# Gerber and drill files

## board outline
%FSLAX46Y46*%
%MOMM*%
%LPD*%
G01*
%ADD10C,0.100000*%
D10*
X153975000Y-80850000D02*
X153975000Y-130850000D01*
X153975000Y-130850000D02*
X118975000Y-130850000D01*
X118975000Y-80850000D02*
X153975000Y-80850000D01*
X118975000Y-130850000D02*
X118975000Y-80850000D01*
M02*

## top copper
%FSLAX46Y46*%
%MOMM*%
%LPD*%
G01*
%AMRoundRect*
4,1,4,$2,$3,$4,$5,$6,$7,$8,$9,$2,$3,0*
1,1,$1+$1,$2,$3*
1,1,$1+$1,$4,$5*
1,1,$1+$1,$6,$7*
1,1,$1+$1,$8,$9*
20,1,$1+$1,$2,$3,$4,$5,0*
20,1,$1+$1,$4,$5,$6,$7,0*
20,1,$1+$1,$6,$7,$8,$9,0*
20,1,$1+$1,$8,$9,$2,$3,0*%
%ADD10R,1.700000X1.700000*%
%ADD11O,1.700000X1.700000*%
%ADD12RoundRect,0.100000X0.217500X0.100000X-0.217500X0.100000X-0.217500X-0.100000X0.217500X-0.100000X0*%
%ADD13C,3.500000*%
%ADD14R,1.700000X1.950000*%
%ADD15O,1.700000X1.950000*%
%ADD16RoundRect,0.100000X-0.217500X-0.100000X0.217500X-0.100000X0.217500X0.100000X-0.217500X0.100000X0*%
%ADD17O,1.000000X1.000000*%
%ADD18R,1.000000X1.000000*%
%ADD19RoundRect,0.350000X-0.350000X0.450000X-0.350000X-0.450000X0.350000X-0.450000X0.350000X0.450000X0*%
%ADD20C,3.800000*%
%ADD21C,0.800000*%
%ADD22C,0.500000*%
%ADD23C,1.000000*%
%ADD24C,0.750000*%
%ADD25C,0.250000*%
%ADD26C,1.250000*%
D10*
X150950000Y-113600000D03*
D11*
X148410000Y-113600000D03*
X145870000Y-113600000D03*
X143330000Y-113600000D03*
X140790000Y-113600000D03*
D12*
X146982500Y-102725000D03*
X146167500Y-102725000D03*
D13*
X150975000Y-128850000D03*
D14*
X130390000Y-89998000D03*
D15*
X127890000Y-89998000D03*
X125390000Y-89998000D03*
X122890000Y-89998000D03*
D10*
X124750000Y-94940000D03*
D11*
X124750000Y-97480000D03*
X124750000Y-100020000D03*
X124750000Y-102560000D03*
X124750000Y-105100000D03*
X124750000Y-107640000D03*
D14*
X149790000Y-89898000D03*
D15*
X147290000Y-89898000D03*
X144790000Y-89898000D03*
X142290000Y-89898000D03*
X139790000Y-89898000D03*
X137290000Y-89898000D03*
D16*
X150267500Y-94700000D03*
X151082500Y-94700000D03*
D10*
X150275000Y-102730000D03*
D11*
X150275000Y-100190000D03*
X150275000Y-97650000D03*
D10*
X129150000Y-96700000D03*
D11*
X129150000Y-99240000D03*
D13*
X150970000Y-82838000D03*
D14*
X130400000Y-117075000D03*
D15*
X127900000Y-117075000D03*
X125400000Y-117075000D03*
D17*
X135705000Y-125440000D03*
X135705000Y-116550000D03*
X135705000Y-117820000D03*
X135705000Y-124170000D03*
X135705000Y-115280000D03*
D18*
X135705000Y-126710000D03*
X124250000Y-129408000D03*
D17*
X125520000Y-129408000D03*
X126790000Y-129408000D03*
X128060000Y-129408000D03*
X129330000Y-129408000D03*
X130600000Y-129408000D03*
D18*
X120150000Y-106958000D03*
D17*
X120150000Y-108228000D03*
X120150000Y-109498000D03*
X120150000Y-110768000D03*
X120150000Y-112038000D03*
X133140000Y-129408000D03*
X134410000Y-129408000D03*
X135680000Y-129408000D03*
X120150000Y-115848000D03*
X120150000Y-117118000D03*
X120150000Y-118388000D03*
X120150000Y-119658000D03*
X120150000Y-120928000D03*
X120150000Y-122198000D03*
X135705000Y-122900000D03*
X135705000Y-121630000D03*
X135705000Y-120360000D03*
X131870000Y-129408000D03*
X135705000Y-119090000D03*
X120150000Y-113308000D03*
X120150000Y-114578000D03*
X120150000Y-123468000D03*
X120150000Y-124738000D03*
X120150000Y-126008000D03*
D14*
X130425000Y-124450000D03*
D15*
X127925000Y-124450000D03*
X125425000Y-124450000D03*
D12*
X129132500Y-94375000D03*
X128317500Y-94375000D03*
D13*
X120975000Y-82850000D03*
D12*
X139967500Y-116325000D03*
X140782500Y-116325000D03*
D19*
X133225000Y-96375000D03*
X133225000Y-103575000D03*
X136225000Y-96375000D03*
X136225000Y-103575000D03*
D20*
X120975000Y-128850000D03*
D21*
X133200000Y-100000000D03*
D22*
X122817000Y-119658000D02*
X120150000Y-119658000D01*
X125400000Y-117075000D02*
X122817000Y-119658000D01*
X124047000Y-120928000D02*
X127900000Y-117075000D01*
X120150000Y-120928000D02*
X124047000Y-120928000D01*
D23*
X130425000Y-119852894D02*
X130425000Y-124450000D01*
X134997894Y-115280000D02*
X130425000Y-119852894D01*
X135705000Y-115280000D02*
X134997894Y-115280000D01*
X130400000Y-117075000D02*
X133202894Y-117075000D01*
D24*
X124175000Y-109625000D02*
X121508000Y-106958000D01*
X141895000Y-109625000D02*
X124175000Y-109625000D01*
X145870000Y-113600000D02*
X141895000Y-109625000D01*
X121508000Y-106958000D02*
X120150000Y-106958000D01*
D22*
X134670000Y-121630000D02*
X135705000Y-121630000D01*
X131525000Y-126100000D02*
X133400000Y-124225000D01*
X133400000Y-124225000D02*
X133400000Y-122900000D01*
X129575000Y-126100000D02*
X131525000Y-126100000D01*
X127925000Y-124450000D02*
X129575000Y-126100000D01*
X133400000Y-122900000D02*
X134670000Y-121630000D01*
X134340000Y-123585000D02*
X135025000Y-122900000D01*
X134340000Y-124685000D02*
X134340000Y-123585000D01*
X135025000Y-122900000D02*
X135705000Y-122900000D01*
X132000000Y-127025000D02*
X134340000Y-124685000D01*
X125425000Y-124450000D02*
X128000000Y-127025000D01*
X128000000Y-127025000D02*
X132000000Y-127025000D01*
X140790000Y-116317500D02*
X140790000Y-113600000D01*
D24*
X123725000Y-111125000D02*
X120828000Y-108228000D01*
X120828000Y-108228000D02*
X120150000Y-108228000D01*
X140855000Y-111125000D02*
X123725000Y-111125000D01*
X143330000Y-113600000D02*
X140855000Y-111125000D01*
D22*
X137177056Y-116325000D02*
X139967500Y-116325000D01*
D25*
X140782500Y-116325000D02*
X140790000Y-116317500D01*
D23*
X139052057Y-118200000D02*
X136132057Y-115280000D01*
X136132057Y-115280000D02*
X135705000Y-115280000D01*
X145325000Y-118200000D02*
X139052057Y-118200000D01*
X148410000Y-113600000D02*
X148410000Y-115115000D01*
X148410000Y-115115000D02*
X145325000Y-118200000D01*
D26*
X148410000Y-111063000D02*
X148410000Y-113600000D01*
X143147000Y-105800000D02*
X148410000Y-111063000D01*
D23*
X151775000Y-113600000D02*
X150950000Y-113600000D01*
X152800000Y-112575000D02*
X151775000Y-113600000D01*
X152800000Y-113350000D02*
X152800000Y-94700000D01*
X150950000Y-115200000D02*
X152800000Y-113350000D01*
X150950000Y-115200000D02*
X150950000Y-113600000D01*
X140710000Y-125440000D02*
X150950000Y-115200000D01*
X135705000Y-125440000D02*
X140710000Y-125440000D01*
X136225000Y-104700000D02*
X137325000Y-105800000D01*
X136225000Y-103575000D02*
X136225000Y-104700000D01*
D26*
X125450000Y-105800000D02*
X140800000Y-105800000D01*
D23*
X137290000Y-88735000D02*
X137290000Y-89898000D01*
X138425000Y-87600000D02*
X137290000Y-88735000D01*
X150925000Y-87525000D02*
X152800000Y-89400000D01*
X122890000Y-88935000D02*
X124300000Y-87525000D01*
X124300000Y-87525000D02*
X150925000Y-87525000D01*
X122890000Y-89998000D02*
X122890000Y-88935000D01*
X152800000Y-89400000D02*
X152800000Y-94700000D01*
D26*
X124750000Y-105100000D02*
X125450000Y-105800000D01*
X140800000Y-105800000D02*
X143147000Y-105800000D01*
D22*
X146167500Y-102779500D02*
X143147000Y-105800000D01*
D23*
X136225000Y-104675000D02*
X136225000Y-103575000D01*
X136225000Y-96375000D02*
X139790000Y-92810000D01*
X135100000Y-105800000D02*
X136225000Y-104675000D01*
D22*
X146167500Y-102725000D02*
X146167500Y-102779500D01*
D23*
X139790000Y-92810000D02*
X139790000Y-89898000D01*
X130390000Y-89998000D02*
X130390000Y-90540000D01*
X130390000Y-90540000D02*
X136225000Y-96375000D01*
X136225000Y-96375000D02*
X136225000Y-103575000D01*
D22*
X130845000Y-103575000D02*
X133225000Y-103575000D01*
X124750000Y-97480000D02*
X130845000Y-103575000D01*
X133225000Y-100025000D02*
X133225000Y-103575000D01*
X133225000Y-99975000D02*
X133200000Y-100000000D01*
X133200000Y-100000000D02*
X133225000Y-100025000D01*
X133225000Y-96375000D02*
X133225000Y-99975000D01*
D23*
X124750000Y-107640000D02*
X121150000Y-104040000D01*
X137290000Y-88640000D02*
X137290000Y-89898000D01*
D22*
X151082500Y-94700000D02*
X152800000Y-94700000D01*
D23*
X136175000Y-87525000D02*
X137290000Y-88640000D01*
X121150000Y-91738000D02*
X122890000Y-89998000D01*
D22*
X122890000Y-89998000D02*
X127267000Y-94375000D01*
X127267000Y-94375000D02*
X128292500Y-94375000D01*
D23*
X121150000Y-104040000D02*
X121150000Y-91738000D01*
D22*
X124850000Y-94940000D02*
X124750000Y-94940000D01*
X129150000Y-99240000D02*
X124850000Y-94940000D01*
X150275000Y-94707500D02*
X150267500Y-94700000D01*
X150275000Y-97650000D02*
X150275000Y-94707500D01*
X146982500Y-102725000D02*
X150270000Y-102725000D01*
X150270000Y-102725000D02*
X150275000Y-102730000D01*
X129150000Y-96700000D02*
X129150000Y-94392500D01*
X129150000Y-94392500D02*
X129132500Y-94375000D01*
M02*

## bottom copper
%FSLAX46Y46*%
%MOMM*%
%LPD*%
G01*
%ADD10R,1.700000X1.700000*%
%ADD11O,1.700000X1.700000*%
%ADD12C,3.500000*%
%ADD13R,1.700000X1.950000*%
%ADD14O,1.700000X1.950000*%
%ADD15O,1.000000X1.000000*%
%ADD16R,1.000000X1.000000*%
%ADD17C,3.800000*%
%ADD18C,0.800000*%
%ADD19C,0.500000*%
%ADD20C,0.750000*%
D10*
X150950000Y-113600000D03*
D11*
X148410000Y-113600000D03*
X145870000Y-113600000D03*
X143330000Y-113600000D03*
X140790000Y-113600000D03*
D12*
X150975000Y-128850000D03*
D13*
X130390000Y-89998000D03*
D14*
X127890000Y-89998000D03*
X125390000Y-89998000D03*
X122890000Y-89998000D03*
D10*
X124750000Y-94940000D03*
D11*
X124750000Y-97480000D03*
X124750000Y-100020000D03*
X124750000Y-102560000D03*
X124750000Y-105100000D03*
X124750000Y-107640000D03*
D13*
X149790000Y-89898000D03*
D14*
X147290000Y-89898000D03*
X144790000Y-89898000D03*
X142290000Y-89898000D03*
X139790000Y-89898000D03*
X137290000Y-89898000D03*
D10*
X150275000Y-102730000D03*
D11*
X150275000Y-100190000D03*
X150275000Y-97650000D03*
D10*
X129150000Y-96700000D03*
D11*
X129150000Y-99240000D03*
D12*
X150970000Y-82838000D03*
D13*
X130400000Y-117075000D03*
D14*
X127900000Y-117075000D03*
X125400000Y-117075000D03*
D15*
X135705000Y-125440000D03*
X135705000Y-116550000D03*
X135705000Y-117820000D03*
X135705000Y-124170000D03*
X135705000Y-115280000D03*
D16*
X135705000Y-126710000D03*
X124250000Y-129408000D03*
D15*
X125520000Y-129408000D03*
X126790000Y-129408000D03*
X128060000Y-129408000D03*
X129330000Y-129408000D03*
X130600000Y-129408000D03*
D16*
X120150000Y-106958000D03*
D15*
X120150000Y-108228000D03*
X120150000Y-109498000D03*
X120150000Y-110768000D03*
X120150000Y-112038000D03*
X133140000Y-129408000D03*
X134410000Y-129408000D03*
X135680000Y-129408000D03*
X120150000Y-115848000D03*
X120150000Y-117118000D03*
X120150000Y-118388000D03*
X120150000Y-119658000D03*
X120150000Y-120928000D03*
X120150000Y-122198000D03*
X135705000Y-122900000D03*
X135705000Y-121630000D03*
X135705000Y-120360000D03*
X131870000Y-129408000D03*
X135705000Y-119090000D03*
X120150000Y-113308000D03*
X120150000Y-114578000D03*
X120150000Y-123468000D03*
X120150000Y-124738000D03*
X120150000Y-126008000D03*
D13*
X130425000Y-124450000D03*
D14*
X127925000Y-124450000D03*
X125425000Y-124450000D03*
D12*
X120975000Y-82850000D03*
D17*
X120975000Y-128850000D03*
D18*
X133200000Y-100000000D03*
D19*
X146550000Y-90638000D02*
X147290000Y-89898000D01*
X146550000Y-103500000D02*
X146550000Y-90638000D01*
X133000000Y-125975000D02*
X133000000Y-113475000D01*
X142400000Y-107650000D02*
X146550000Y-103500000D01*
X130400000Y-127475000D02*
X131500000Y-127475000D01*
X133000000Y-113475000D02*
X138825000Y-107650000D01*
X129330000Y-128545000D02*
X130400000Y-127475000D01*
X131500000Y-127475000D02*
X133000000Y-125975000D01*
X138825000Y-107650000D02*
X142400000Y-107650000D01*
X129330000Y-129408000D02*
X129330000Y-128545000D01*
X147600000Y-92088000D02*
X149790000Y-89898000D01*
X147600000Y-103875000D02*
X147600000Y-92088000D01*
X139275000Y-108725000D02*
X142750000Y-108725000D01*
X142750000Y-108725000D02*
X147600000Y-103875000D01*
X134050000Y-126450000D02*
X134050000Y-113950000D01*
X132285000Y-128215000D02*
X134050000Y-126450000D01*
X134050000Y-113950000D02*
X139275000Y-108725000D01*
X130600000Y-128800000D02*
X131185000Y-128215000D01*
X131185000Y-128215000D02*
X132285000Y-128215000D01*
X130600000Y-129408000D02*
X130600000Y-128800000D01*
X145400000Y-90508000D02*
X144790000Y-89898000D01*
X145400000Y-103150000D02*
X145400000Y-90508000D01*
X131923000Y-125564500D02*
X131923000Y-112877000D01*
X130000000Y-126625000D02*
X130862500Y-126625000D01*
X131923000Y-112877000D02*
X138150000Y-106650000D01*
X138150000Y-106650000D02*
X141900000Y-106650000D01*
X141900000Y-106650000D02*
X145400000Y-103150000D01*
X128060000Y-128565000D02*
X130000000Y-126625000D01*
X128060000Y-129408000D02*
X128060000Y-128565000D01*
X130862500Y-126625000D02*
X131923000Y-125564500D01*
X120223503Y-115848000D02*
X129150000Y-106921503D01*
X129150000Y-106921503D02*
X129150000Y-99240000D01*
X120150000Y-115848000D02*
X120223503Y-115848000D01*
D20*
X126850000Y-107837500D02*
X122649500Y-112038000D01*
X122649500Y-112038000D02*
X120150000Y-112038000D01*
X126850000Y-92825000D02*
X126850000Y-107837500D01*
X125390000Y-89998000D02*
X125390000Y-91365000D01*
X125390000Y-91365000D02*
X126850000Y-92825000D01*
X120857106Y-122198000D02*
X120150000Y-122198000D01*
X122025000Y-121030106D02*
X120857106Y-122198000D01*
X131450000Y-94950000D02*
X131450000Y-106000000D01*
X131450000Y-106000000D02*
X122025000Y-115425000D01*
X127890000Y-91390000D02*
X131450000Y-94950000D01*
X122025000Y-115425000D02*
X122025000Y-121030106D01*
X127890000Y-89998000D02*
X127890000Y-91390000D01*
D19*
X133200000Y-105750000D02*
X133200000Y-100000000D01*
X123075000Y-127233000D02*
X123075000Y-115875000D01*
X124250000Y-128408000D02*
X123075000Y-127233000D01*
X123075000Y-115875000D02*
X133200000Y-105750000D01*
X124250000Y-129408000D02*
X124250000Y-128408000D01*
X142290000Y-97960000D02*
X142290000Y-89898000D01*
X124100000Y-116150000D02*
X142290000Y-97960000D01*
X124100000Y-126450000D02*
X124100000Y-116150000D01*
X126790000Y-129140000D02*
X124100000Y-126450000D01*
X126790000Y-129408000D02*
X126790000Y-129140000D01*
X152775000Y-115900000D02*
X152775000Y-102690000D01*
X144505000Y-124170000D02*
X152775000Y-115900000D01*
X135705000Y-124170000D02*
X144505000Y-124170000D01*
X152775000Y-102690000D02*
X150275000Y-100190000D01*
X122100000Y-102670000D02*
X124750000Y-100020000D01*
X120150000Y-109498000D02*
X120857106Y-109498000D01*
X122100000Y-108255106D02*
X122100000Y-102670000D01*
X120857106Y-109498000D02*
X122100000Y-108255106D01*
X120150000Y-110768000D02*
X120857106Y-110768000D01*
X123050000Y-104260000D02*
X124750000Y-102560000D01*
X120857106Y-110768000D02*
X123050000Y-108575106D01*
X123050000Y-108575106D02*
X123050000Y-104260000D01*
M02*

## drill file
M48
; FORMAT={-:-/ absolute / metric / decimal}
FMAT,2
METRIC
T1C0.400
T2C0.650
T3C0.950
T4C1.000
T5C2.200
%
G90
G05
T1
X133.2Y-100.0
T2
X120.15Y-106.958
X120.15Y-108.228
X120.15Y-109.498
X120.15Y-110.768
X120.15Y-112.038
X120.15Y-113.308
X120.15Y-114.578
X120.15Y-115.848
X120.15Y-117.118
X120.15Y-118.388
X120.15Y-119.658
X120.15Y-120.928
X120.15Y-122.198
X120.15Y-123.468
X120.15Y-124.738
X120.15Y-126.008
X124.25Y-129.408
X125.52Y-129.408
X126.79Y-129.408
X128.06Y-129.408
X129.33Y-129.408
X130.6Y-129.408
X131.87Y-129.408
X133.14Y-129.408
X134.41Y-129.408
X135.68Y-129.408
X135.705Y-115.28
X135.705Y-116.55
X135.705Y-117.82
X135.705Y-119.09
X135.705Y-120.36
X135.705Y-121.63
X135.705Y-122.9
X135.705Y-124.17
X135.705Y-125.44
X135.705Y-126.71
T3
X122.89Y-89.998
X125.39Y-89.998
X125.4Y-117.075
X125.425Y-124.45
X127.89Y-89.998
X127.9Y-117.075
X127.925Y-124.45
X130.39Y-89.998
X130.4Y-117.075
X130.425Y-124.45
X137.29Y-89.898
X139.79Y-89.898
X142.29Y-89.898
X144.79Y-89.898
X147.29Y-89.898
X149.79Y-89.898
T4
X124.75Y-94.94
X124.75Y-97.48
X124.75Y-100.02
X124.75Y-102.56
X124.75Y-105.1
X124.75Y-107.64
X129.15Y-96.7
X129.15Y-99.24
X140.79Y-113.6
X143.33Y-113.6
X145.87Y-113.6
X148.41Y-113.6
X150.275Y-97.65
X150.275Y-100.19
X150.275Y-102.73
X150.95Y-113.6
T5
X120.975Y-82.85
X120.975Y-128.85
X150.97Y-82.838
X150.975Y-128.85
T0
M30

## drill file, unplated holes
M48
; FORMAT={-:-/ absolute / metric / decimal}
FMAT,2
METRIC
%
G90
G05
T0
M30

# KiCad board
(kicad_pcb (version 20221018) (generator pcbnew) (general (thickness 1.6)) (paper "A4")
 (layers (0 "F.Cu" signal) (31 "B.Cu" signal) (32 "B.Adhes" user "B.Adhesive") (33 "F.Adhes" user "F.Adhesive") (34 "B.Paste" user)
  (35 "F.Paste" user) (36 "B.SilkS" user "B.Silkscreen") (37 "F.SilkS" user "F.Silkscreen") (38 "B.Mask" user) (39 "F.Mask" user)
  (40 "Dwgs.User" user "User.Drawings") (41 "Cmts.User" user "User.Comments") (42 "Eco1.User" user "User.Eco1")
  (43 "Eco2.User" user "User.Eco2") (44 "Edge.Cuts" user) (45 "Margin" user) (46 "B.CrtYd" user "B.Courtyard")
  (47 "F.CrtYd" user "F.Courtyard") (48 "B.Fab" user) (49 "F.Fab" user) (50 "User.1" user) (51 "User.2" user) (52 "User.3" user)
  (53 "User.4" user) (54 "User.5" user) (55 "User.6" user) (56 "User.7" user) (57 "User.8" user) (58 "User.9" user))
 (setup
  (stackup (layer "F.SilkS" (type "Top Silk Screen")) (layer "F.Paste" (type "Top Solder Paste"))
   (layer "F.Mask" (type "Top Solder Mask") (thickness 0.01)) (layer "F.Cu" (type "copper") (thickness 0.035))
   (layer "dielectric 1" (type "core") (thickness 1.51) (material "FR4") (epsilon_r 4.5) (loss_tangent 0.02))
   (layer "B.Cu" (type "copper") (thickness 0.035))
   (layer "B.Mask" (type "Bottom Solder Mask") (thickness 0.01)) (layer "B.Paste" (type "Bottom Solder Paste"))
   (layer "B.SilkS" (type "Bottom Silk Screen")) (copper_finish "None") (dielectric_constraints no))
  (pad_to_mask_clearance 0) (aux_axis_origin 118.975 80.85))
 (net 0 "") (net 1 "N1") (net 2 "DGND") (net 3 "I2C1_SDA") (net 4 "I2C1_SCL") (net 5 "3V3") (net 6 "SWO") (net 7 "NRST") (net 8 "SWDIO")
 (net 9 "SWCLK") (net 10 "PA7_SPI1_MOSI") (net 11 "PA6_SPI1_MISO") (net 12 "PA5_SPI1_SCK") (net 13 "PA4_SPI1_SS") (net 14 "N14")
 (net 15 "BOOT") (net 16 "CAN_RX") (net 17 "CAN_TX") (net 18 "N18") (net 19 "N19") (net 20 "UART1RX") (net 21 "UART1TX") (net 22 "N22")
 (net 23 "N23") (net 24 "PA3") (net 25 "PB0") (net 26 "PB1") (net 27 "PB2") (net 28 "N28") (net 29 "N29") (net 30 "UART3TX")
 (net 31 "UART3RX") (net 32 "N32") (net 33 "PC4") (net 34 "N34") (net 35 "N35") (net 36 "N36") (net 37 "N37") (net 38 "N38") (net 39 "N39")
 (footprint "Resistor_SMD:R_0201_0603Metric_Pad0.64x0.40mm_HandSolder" (layer "F.Cu") (at 146.575 102.725 180)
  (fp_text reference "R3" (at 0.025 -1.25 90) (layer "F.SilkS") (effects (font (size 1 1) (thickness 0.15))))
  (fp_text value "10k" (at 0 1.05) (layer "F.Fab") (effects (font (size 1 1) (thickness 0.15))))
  (pad "" smd roundrect (at -0.4325 0 180) (size 0.458 0.36) (layers "F.Paste") (roundrect_rratio 0.25))
  (pad "" smd roundrect (at 0.4325 0 180) (size 0.458 0.36) (layers "F.Paste") (roundrect_rratio 0.25))
  (pad "1" smd roundrect (at -0.4075 0 180) (size 0.635 0.4) (layers "F.Cu" "F.Mask") (roundrect_rratio 0.25) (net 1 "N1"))
  (pad "2" smd roundrect (at 0.4075 0 180) (size 0.635 0.4) (layers "F.Cu" "F.Mask") (roundrect_rratio 0.25) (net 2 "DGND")))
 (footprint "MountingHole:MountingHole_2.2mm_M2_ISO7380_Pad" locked (layer "F.Cu") (at 150.975 128.85)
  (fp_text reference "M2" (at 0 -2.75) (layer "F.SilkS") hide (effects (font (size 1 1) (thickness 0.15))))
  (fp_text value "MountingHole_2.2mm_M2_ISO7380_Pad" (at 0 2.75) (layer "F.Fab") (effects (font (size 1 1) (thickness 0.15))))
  (pad "1" thru_hole circle locked (at 0 0) (size 3.5 3.5) (drill 2.2) (layers "*.Cu" "*.Mask")))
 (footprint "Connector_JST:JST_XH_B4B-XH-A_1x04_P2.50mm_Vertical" (layer "F.Cu") (at 130.39 89.998 180)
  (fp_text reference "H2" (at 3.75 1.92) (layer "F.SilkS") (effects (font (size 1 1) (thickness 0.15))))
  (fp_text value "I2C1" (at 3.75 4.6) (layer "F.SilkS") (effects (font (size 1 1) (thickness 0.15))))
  (pad "1" thru_hole rect (at 0 0 180) (size 1.7 1.95) (drill 0.95) (layers "*.Cu" "*.Mask") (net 2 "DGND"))
  (pad "2" thru_hole oval (at 2.5 0 180) (size 1.7 1.95) (drill 0.95) (layers "*.Cu" "*.Mask") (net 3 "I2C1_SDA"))
  (pad "3" thru_hole oval (at 5 0 180) (size 1.7 1.95) (drill 0.95) (layers "*.Cu" "*.Mask") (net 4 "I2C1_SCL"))
  (pad "4" thru_hole oval (at 7.5 0 180) (size 1.7 1.95) (drill 0.95) (layers "*.Cu" "*.Mask") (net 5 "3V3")))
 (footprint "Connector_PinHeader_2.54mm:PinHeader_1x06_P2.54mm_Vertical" (layer "F.Cu") (at 124.75 94.94)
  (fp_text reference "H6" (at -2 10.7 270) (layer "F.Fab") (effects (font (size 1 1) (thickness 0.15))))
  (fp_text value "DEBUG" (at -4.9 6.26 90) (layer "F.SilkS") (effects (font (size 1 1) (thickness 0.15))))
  (pad "1" thru_hole rect (at 0 0) (size 1.7 1.7) (drill 1) (layers "*.Cu" "*.Mask") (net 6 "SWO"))
  (pad "2" thru_hole oval (at 0 2.54) (size 1.7 1.7) (drill 1) (layers "*.Cu" "*.Mask") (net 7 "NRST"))
  (pad "3" thru_hole oval (at 0 5.08) (size 1.7 1.7) (drill 1) (layers "*.Cu" "*.Mask") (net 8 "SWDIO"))
  (pad "4" thru_hole oval (at 0 7.62) (size 1.7 1.7) (drill 1) (layers "*.Cu" "*.Mask") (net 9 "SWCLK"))
  (pad "5" thru_hole oval (at 0 10.16) (size 1.7 1.7) (drill 1) (layers "*.Cu" "*.Mask") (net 2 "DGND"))
  (pad "6" thru_hole oval (at 0 12.7) (size 1.7 1.7) (drill 1) (layers "*.Cu" "*.Mask") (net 5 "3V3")))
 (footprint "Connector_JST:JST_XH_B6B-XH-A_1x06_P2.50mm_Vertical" (layer "F.Cu") (at 149.79 89.898 180)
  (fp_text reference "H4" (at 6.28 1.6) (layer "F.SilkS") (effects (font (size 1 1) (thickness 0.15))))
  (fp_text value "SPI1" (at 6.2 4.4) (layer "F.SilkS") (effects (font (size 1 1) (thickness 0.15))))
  (pad "1" thru_hole rect (at 0 0 180) (size 1.7 1.95) (drill 0.95) (layers "*.Cu" "*.Mask") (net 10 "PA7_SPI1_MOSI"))
  (pad "2" thru_hole oval (at 2.5 0 180) (size 1.7 1.95) (drill 0.95) (layers "*.Cu" "*.Mask") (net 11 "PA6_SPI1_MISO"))
  (pad "3" thru_hole oval (at 5 0 180) (size 1.7 1.95) (drill 0.95) (layers "*.Cu" "*.Mask") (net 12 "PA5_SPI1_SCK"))
  (pad "4" thru_hole oval (at 7.5 0 180) (size 1.7 1.95) (drill 0.95) (layers "*.Cu" "*.Mask") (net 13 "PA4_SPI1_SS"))
  (pad "5" thru_hole oval (at 10 0 180) (size 1.7 1.95) (drill 0.95) (layers "*.Cu" "*.Mask") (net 2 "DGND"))
  (pad "6" thru_hole oval (at 12.5 0 180) (size 1.7 1.95) (drill 0.95) (layers "*.Cu" "*.Mask") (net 5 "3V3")))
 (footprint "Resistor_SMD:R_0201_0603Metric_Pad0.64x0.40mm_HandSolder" (layer "F.Cu") (at 150.675 94.7)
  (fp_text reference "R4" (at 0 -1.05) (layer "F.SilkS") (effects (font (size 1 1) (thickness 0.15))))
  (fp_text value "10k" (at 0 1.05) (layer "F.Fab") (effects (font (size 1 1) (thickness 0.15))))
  (pad "" smd roundrect (at -0.4325 0) (size 0.458 0.36) (layers "F.Paste") (roundrect_rratio 0.25))
  (pad "" smd roundrect (at 0.4325 0) (size 0.458 0.36) (layers "F.Paste") (roundrect_rratio 0.25))
  (pad "1" smd roundrect (at -0.4075 0) (size 0.635 0.4) (layers "F.Cu" "F.Mask") (roundrect_rratio 0.25) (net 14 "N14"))
  (pad "2" smd roundrect (at 0.4075 0) (size 0.635 0.4) (layers "F.Cu" "F.Mask") (roundrect_rratio 0.25) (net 5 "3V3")))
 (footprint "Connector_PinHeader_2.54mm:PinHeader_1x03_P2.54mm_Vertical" (layer "F.Cu") (at 150.275 102.73 180)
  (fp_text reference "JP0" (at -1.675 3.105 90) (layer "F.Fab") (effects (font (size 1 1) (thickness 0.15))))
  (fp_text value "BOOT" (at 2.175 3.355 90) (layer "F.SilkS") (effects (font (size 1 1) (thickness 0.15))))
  (pad "1" thru_hole rect (at 0 0 180) (size 1.7 1.7) (drill 1) (layers "*.Cu" "*.Mask") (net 1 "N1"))
  (pad "2" thru_hole oval (at 0 2.54 180) (size 1.7 1.7) (drill 1) (layers "*.Cu" "*.Mask") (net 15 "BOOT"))
  (pad "3" thru_hole oval (at 0 5.08 180) (size 1.7 1.7) (drill 1) (layers "*.Cu" "*.Mask") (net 14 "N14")))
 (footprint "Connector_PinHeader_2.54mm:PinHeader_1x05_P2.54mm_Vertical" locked (layer "F.Cu") (at 150.95 113.6 -90)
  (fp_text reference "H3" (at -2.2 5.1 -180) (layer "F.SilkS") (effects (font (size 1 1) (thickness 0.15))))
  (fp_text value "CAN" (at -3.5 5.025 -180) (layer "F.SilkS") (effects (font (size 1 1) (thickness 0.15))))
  (pad "1" thru_hole rect locked (at 0 0 270) (size 1.7 1.7) (drill 1) (layers "*.Cu" "*.Mask") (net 5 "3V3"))
  (pad "2" thru_hole oval locked (at 0 2.54 270) (size 1.7 1.7) (drill 1) (layers "*.Cu" "*.Mask") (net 2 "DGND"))
  (pad "3" thru_hole oval locked (at 0 5.08 270) (size 1.7 1.7) (drill 1) (layers "*.Cu" "*.Mask") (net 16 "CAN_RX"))
  (pad "4" thru_hole oval locked (at 0 7.62 270) (size 1.7 1.7) (drill 1) (layers "*.Cu" "*.Mask") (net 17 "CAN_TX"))
  (pad "5" thru_hole oval locked (at 0 10.16 270) (size 1.7 1.7) (drill 1) (layers "*.Cu" "*.Mask") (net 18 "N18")))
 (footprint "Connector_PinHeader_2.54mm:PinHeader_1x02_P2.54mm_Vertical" (layer "F.Cu") (at 129.15 96.7)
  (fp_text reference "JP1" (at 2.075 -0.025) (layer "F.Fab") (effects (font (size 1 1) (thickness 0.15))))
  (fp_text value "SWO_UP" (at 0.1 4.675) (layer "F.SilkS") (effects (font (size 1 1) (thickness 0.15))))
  (pad "1" thru_hole rect (at 0 0) (size 1.7 1.7) (drill 1) (layers "*.Cu" "*.Mask") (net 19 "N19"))
  (pad "2" thru_hole oval (at 0 2.54) (size 1.7 1.7) (drill 1) (layers "*.Cu" "*.Mask") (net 6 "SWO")))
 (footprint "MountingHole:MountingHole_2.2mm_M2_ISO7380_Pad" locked (layer "F.Cu") (at 150.97 82.838)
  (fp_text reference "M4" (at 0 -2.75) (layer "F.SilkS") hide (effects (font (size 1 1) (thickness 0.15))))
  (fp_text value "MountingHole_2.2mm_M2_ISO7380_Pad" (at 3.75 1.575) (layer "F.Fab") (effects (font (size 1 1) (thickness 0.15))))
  (pad "1" thru_hole circle locked (at 0 0) (size 3.5 3.5) (drill 2.2) (layers "*.Cu" "*.Mask")))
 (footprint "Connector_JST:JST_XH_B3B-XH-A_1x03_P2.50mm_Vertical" (layer "F.Cu") (at 130.4 117.075 180)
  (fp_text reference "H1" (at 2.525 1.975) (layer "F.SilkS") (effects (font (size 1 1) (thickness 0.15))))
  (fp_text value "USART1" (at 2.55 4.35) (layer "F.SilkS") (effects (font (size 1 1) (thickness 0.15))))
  (pad "1" thru_hole rect (at 0 0 180) (size 1.7 1.95) (drill 0.95) (layers "*.Cu" "*.Mask") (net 2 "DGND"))
  (pad "2" thru_hole oval (at 2.5 0 180) (size 1.7 1.95) (drill 0.95) (layers "*.Cu" "*.Mask") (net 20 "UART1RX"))
  (pad "3" thru_hole oval (at 5 0 180) (size 1.7 1.95) (drill 0.95) (layers "*.Cu" "*.Mask") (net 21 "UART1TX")))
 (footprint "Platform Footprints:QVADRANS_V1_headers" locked (layer "F.Cu") (at 120.15 126.008)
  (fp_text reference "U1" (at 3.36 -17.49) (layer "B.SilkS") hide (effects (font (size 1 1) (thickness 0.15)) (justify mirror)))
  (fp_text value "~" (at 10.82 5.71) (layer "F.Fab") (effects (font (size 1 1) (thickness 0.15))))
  (pad "3V3" thru_hole oval locked (at 15.555 -0.568 180) (size 1 1) (drill 0.65) (layers "*.Cu" "*.Mask") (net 5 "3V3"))
  (pad "5V" thru_hole oval locked (at 15.555 -9.458 180) (size 1 1) (drill 0.65) (layers "*.Cu" "*.Mask") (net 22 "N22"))
  (pad "12V" thru_hole oval locked (at 15.555 -8.188 180) (size 1 1) (drill 0.65) (layers "*.Cu" "*.Mask") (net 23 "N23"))
  (pad "BOOT" thru_hole oval locked (at 15.555 -1.838 180) (size 1 1) (drill 0.65) (layers "*.Cu" "*.Mask") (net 15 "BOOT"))
  (pad "DGND" thru_hole oval locked (at 15.555 -10.728 180) (size 1 1) (drill 0.65) (layers "*.Cu" "*.Mask") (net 2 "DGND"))
  (pad "DGND" thru_hole rect locked (at 15.555 0.702 180) (size 1 1) (drill 0.65) (layers "*.Cu" "*.Mask") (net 2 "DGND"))
  (pad "NRST" thru_hole rect locked (at 4.1 3.4 90) (size 1 1) (drill 0.65) (layers "*.Cu" "*.Mask") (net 7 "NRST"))
  (pad "PA3" thru_hole oval locked (at 5.37 3.4 90) (size 1 1) (drill 0.65) (layers "*.Cu" "*.Mask") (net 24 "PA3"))
  (pad "PA4" thru_hole oval locked (at 6.64 3.4 90) (size 1 1) (drill 0.65) (layers "*.Cu" "*.Mask") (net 13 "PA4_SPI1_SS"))
  (pad "PA5" thru_hole oval locked (at 7.91 3.4 90) (size 1 1) (drill 0.65) (layers "*.Cu" "*.Mask") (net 12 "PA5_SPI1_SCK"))
  (pad "PA6" thru_hole oval locked (at 9.18 3.4 90) (size 1 1) (drill 0.65) (layers "*.Cu" "*.Mask") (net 11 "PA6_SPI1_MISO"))
  (pad "PA7" thru_hole oval locked (at 10.45 3.4 90) (size 1 1) (drill 0.65) (layers "*.Cu" "*.Mask") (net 10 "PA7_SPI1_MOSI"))
  (pad "PA11" thru_hole rect locked (at 0 -19.05) (size 1 1) (drill 0.65) (layers "*.Cu" "*.Mask") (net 16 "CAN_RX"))
  (pad "PA12" thru_hole oval locked (at 0 -17.78) (size 1 1) (drill 0.65) (layers "*.Cu" "*.Mask") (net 17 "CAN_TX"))
  (pad "PA13" thru_hole oval locked (at 0 -16.51) (size 1 1) (drill 0.65) (layers "*.Cu" "*.Mask") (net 8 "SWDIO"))
  (pad "PA14" thru_hole oval locked (at 0 -15.24) (size 1 1) (drill 0.65) (layers "*.Cu" "*.Mask") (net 9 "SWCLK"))
  (pad "PA15" thru_hole oval locked (at 0 -13.97) (size 1 1) (drill 0.65) (layers "*.Cu" "*.Mask") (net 4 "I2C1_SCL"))
  (pad "PB0" thru_hole oval locked (at 12.99 3.4 90) (size 1 1) (drill 0.65) (layers "*.Cu" "*.Mask") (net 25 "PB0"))
  (pad "PB1" thru_hole oval locked (at 14.26 3.4 90) (size 1 1) (drill 0.65) (layers "*.Cu" "*.Mask") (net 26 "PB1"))
  (pad "PB2" thru_hole oval locked (at 15.53 3.4 90) (size 1 1) (drill 0.65) (layers "*.Cu" "*.Mask") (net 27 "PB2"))
  (pad "PB3" thru_hole oval locked (at 0 -10.16) (size 1 1) (drill 0.65) (layers "*.Cu" "*.Mask") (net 6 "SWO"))
  (pad "PB4" thru_hole oval locked (at 0 -8.89) (size 1 1) (drill 0.65) (layers "*.Cu" "*.Mask") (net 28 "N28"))
  (pad "PB5" thru_hole oval locked (at 0 -7.62) (size 1 1) (drill 0.65) (layers "*.Cu" "*.Mask") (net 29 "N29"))
  (pad "PB6" thru_hole oval locked (at 0 -6.35) (size 1 1) (drill 0.65) (layers "*.Cu" "*.Mask") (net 21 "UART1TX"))
  (pad "PB7" thru_hole oval locked (at 0 -5.08) (size 1 1) (drill 0.65) (layers "*.Cu" "*.Mask") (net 20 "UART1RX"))
  (pad "PB9" thru_hole oval locked (at 0 -3.81) (size 1 1) (drill 0.65) (layers "*.Cu" "*.Mask") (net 3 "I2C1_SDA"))
  (pad "PB10" thru_hole oval locked (at 15.555 -3.108 180) (size 1 1) (drill 0.65) (layers "*.Cu" "*.Mask") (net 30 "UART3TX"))
  (pad "PB11" thru_hole oval locked (at 15.555 -4.378 180) (size 1 1) (drill 0.65) (layers "*.Cu" "*.Mask") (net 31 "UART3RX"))
  (pad "PB12" thru_hole oval locked (at 15.555 -5.648 180) (size 1 1) (drill 0.65) (layers "*.Cu" "*.Mask") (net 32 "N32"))
  (pad "PC4" thru_hole oval locked (at 11.72 3.4 90) (size 1 1) (drill 0.65) (layers "*.Cu" "*.Mask") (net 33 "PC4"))
  (pad "PC6" thru_hole oval locked (at 15.555 -6.918 180) (size 1 1) (drill 0.65) (layers "*.Cu" "*.Mask") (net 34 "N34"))
  (pad "PC10" thru_hole oval locked (at 0 -12.7) (size 1 1) (drill 0.65) (layers "*.Cu" "*.Mask") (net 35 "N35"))
  (pad "PC11" thru_hole oval locked (at 0 -11.43) (size 1 1) (drill 0.65) (layers "*.Cu" "*.Mask") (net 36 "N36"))
  (pad "PC13" thru_hole oval locked (at 0 -2.54) (size 1 1) (drill 0.65) (layers "*.Cu" "*.Mask") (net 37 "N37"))
  (pad "PC14" thru_hole oval locked (at 0 -1.27) (size 1 1) (drill 0.65) (layers "*.Cu" "*.Mask") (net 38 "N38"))
  (pad "PC15" thru_hole oval locked (at 0 0) (size 1 1) (drill 0.65) (layers "*.Cu" "*.Mask") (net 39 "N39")))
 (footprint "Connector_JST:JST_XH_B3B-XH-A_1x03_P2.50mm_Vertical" (layer "F.Cu") (at 130.425 124.45 180)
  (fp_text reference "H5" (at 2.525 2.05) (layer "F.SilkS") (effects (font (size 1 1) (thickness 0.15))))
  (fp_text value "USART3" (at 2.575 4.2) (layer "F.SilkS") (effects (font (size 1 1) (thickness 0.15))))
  (pad "1" thru_hole rect (at 0 0 180) (size 1.7 1.95) (drill 0.95) (layers "*.Cu" "*.Mask") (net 2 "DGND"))
  (pad "2" thru_hole oval (at 2.5 0 180) (size 1.7 1.95) (drill 0.95) (layers "*.Cu" "*.Mask") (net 31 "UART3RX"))
  (pad "3" thru_hole oval (at 5 0 180) (size 1.7 1.95) (drill 0.95) (layers "*.Cu" "*.Mask") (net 30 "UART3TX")))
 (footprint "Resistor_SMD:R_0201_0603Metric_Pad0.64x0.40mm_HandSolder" (layer "F.Cu") (at 128.725 94.375 180)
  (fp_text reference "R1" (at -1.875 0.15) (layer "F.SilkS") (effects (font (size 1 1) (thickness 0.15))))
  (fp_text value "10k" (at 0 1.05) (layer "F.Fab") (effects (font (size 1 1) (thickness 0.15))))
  (pad "" smd roundrect (at -0.4325 0 180) (size 0.458 0.36) (layers "F.Paste") (roundrect_rratio 0.25))
  (pad "" smd roundrect (at 0.4325 0 180) (size 0.458 0.36) (layers "F.Paste") (roundrect_rratio 0.25))
  (pad "1" smd roundrect (at -0.4075 0 180) (size 0.635 0.4) (layers "F.Cu" "F.Mask") (roundrect_rratio 0.25) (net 19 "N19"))
  (pad "2" smd roundrect (at 0.4075 0 180) (size 0.635 0.4) (layers "F.Cu" "F.Mask") (roundrect_rratio 0.25) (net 5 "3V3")))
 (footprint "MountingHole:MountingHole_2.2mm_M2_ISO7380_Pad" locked (layer "F.Cu") (at 120.975 82.85)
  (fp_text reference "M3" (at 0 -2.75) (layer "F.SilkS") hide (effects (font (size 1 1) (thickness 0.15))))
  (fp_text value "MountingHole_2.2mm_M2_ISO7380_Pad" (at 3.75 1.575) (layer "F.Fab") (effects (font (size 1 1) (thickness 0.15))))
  (pad "1" thru_hole circle locked (at 0 0) (size 3.5 3.5) (drill 2.2) (layers "*.Cu" "*.Mask")))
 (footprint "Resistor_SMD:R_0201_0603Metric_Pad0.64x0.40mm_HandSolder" (layer "F.Cu") (at 140.375 116.325 180)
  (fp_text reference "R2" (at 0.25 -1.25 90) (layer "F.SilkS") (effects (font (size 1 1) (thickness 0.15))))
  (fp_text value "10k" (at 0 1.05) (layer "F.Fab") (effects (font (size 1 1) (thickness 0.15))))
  (pad "" smd roundrect (at -0.4325 0 180) (size 0.458 0.36) (layers "F.Paste") (roundrect_rratio 0.25))
  (pad "" smd roundrect (at 0.4325 0 180) (size 0.458 0.36) (layers "F.Paste") (roundrect_rratio 0.25))
  (pad "1" smd roundrect (at -0.4075 0 180) (size 0.635 0.4) (layers "F.Cu" "F.Mask") (roundrect_rratio 0.25) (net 18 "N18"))
  (pad "2" smd roundrect (at 0.4075 0 180) (size 0.635 0.4) (layers "F.Cu" "F.Mask") (roundrect_rratio 0.25) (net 2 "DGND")))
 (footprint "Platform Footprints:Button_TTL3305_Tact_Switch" (layer "F.Cu") (at 134.725 99.975 -90)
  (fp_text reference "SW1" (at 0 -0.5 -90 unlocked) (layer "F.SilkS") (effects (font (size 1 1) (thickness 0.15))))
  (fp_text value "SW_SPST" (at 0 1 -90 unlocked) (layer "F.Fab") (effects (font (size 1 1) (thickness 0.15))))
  (pad "1" smd roundrect (at -3.6 1.5 270) (size 1.6 1.4) (layers "F.Cu" "F.Paste" "F.Mask") (roundrect_rratio 0.25) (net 7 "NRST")
   (thermal_bridge_angle 45))
  (pad "1" smd roundrect (at 3.6 1.5 270) (size 1.6 1.4) (layers "F.Cu" "F.Paste" "F.Mask") (roundrect_rratio 0.25) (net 7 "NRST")
   (thermal_bridge_angle 45))
  (pad "2" smd roundrect (at -3.6 -1.5 270) (size 1.6 1.4) (layers "F.Cu" "F.Paste" "F.Mask") (roundrect_rratio 0.25) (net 2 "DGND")
   (thermal_bridge_angle 45))
  (pad "2" smd roundrect (at 3.6 -1.5 270) (size 1.6 1.4) (layers "F.Cu" "F.Paste" "F.Mask") (roundrect_rratio 0.25) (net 2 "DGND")
   (thermal_bridge_angle 45)))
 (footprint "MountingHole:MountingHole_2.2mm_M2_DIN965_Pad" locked (layer "F.Cu") (at 120.975 128.85)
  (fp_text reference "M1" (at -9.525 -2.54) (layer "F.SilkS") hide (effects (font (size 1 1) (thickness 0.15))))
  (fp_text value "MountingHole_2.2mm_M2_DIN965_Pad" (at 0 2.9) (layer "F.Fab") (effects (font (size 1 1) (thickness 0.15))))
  (pad "1" thru_hole circle locked (at 0 0) (size 3.8 3.8) (drill 2.2) (layers "*.Cu" "*.Mask")))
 (gr_line (start 153.975 80.85) (end 153.975 130.85) (stroke (width 0.1) (type default)) (layer "Edge.Cuts"))
 (gr_line (start 153.975 130.85) (end 118.975 130.85) (stroke (width 0.1) (type default)) (layer "Edge.Cuts"))
 (gr_line (start 118.975 80.85) (end 153.975 80.85) (stroke (width 0.1) (type default)) (layer "Edge.Cuts"))
 (gr_line (start 118.975 130.85) (end 118.975 80.85) (stroke (width 0.1) (type default)) (layer "Edge.Cuts"))
 (segment (start 139.052057 118.2) (end 136.132057 115.28) (width 1) (layer "F.Cu") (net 2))
 (segment (start 124.75 105.1) (end 125.45 105.8) (width 1.25) (layer "F.Cu") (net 2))
 (segment (start 135.705 115.28) (end 134.997894 115.28) (width 1) (layer "F.Cu") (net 2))
 (segment (start 143.147 105.8) (end 148.41 111.063) (width 1.25) (layer "F.Cu") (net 2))
 (segment (start 148.41 111.063) (end 148.41 113.6) (width 1.25) (layer "F.Cu") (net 2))
 (segment (start 140.8 105.8) (end 143.147 105.8) (width 1.25) (layer "F.Cu") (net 2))
 (segment (start 137.177056 116.325) (end 139.9675 116.325) (width 0.5) (layer "F.Cu") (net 2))
 (segment (start 145.325 118.2) (end 139.052057 118.2) (width 1) (layer "F.Cu") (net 2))
 (segment (start 136.225 104.7) (end 137.325 105.8) (width 1) (layer "F.Cu") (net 2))
 (segment (start 148.41 115.115) (end 145.325 118.2) (width 1) (layer "F.Cu") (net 2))
 (segment (start 130.425 119.852894) (end 130.425 124.45) (width 1) (layer "F.Cu") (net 2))
 (segment (start 148.41 113.6) (end 148.41 115.115) (width 1) (layer "F.Cu") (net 2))
 (segment (start 146.1675 102.7795) (end 143.147 105.8) (width 0.5) (layer "F.Cu") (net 2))
 (segment (start 125.45 105.8) (end 140.8 105.8) (width 1.25) (layer "F.Cu") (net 2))
 (segment (start 136.225 104.675) (end 136.225 103.575) (width 1) (layer "F.Cu") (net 2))
 (segment (start 136.132057 115.28) (end 135.705 115.28) (width 1) (layer "F.Cu") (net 2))
 (segment (start 136.225 103.575) (end 136.225 104.7) (width 1) (layer "F.Cu") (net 2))
 (segment (start 130.4 117.075) (end 133.202894 117.075) (width 1) (layer "F.Cu") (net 2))
 (segment (start 136.225 96.375) (end 139.79 92.81) (width 1) (layer "F.Cu") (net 2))
 (segment (start 135.1 105.8) (end 136.225 104.675) (width 1) (layer "F.Cu") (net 2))
 (segment (start 146.1675 102.725) (end 146.1675 102.7795) (width 0.5) (layer "F.Cu") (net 2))
 (segment (start 139.79 92.81) (end 139.79 89.898) (width 1) (layer "F.Cu") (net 2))
 (segment (start 134.997894 115.28) (end 130.425 119.852894) (width 1) (layer "F.Cu") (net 2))
 (segment (start 130.39 89.998) (end 130.39 90.54) (width 1) (layer "F.Cu") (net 2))
 (segment (start 130.39 90.54) (end 136.225 96.375) (width 1) (layer "F.Cu") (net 2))
 (segment (start 136.225 96.375) (end 136.225 103.575) (width 1) (layer "F.Cu") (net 2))
 (segment (start 130.845 103.575) (end 133.225 103.575) (width 0.5) (layer "F.Cu") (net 7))
 (segment (start 124.75 97.48) (end 130.845 103.575) (width 0.5) (layer "F.Cu") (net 7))
 (segment (start 133.225 100.025) (end 133.225 103.575) (width 0.5) (layer "F.Cu") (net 7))
 (segment (start 133.225 99.975) (end 133.2 100) (width 0.5) (layer "F.Cu") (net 7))
 (segment (start 133.2 100) (end 133.225 100.025) (width 0.5) (layer "F.Cu") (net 7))
 (segment (start 133.225 96.375) (end 133.225 99.975) (width 0.5) (layer "F.Cu") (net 7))
 (via (at 133.2 100) (size 0.8) (drill 0.4) (layers "F.Cu" "B.Cu") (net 7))
 (segment (start 133.2 105.75) (end 133.2 100) (width 0.5) (layer "B.Cu") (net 7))
 (segment (start 123.075 115.875) (end 133.2 105.75) (width 0.5) (layer "B.Cu") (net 7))
 (segment (start 124.25 129.408) (end 124.25 128.408) (width 0.5) (layer "B.Cu") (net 7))
 (segment (start 124.25 128.408) (end 123.075 127.233) (width 0.5) (layer "B.Cu") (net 7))
 (segment (start 123.075 127.233) (end 123.075 115.875) (width 0.5) (layer "B.Cu") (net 7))
 (segment (start 135.705 124.17) (end 144.505 124.17) (width 0.5) (layer "B.Cu") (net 15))
 (segment (start 144.505 124.17) (end 152.775 115.9) (width 0.5) (layer "B.Cu") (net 15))
 (segment (start 152.775 115.9) (end 152.775 102.69) (width 0.5) (layer "B.Cu") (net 15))
 (segment (start 152.775 102.69) (end 150.275 100.19) (width 0.5) (layer "B.Cu") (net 15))
 (segment (start 152.8 89.4) (end 152.8 94.7) (width 1) (layer "F.Cu") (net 5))
 (segment (start 140.71 125.44) (end 150.95 115.2) (width 1) (layer "F.Cu") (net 5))
 (segment (start 124.75 107.64) (end 121.15 104.04) (width 1) (layer "F.Cu") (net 5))
 (segment (start 122.89 89.998) (end 122.89 88.935) (width 1) (layer "F.Cu") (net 5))
 (segment (start 138.425 87.6) (end 137.29 88.735) (width 1) (layer "F.Cu") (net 5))
 (segment (start 137.29 88.64) (end 137.29 89.898) (width 1) (layer "F.Cu") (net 5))
 (segment (start 122.89 88.935) (end 124.3 87.525) (width 1) (layer "F.Cu") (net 5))
 (segment (start 151.775 113.6) (end 150.95 113.6) (width 1) (layer "F.Cu") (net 5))
 (segment (start 151.0825 94.7) (end 152.8 94.7) (width 0.5) (layer "F.Cu") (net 5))
 (segment (start 150.95 115.2) (end 152.8 113.35) (width 1) (layer "F.Cu") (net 5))
 (segment (start 136.175 87.525) (end 137.29 88.64) (width 1) (layer "F.Cu") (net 5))
 (segment (start 152.8 113.35) (end 152.8 94.7) (width 1) (layer "F.Cu") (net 5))
 (segment (start 135.705 125.44) (end 140.71 125.44) (width 1) (layer "F.Cu") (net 5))
 (segment (start 137.29 88.735) (end 137.29 89.898) (width 1) (layer "F.Cu") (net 5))
 (segment (start 150.925 87.525) (end 152.8 89.4) (width 1) (layer "F.Cu") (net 5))
 (segment (start 121.15 91.738) (end 122.89 89.998) (width 1) (layer "F.Cu") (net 5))
 (segment (start 152.8 112.575) (end 151.775 113.6) (width 1) (layer "F.Cu") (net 5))
 (segment (start 122.89 89.998) (end 127.267 94.375) (width 0.5) (layer "F.Cu") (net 5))
 (segment (start 127.267 94.375) (end 128.2925 94.375) (width 0.5) (layer "F.Cu") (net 5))
 (segment (start 121.15 104.04) (end 121.15 91.738) (width 1) (layer "F.Cu") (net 5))
 (segment (start 124.3 87.525) (end 150.925 87.525) (width 1) (layer "F.Cu") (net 5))
 (segment (start 150.95 115.2) (end 150.95 113.6) (width 1) (layer "F.Cu") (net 5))
 (segment (start 125.39 89.998) (end 125.39 91.365) (width 0.75) (layer "B.Cu") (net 4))
 (segment (start 126.85 92.825) (end 126.85 107.8375) (width 0.75) (layer "B.Cu") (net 4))
 (segment (start 125.39 91.365) (end 126.85 92.825) (width 0.75) (layer "B.Cu") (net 4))
 (segment (start 126.85 107.8375) (end 122.6495 112.038) (width 0.75) (layer "B.Cu") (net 4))
 (segment (start 122.6495 112.038) (end 120.15 112.038) (width 0.75) (layer "B.Cu") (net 4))
 (segment (start 131.45 94.95) (end 131.45 106) (width 0.75) (layer "B.Cu") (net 3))
 (segment (start 122.025 115.425) (end 122.025 121.030106) (width 0.75) (layer "B.Cu") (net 3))
 (segment (start 131.45 106) (end 122.025 115.425) (width 0.75) (layer "B.Cu") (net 3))
 (segment (start 122.025 121.030106) (end 120.857106 122.198) (width 0.75) (layer "B.Cu") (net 3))
 (segment (start 127.89 89.998) (end 127.89 91.39) (width 0.75) (layer "B.Cu") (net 3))
 (segment (start 120.857106 122.198) (end 120.15 122.198) (width 0.75) (layer "B.Cu") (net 3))
 (segment (start 127.89 91.39) (end 131.45 94.95) (width 0.75) (layer "B.Cu") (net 3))
 (segment (start 123.725 111.125) (end 120.828 108.228) (width 0.75) (layer "F.Cu") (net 17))
 (segment (start 143.33 113.6) (end 140.855 111.125) (width 0.75) (layer "F.Cu") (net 17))
 (segment (start 120.828 108.228) (end 120.15 108.228) (width 0.75) (layer "F.Cu") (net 17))
 (segment (start 140.855 111.125) (end 123.725 111.125) (width 0.75) (layer "F.Cu") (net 17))
 (segment (start 145.87 113.6) (end 141.895 109.625) (width 0.75) (layer "F.Cu") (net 16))
 (segment (start 121.508 106.958) (end 120.15 106.958) (width 0.75) (layer "F.Cu") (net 16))
 (segment (start 141.895 109.625) (end 124.175 109.625) (width 0.75) (layer "F.Cu") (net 16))
 (segment (start 124.175 109.625) (end 121.508 106.958) (width 0.75) (layer "F.Cu") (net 16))
 (segment (start 122.817 119.658) (end 120.15 119.658) (width 0.5) (layer "F.Cu") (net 21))
 (segment (start 125.4 117.075) (end 122.817 119.658) (width 0.5) (layer "F.Cu") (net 21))
 (segment (start 124.047 120.928) (end 127.9 117.075) (width 0.5) (layer "F.Cu") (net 20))
 (segment (start 120.15 120.928) (end 124.047 120.928) (width 0.5) (layer "F.Cu") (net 20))
 (segment (start 145.4 103.15) (end 145.4 90.508) (width 0.5) (layer "B.Cu") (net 12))
 (segment (start 128.06 128.565) (end 130 126.625) (width 0.5) (layer "B.Cu") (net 12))
 (segment (start 131.923 125.5645) (end 131.923 112.877) (width 0.5) (layer "B.Cu") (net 12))
 (segment (start 128.06 129.408) (end 128.06 128.565) (width 0.5) (layer "B.Cu") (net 12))
 (segment (start 141.9 106.65) (end 145.4 103.15) (width 0.5) (layer "B.Cu") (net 12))
 (segment (start 130.8625 126.625) (end 131.923 125.5645) (width 0.5) (layer "B.Cu") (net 12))
 (segment (start 138.15 106.65) (end 141.9 106.65) (width 0.5) (layer "B.Cu") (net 12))
 (segment (start 130 126.625) (end 130.8625 126.625) (width 0.5) (layer "B.Cu") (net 12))
 (segment (start 131.923 112.877) (end 138.15 106.65) (width 0.5) (layer "B.Cu") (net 12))
 (segment (start 145.4 90.508) (end 144.79 89.898) (width 0.5) (layer "B.Cu") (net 12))
 (segment (start 142.4 107.65) (end 146.55 103.5) (width 0.5) (layer "B.Cu") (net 11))
 (segment (start 133 113.475) (end 138.825 107.65) (width 0.5) (layer "B.Cu") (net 11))
 (segment (start 133 125.975) (end 133 113.475) (width 0.5) (layer "B.Cu") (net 11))
 (segment (start 129.33 128.545) (end 130.4 127.475) (width 0.5) (layer "B.Cu") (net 11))
 (segment (start 138.825 107.65) (end 142.4 107.65) (width 0.5) (layer "B.Cu") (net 11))
 (segment (start 146.55 90.638) (end 147.29 89.898) (width 0.5) (layer "B.Cu") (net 11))
 (segment (start 130.4 127.475) (end 131.5 127.475) (width 0.5) (layer "B.Cu") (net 11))
 (segment (start 146.55 103.5) (end 146.55 90.638) (width 0.5) (layer "B.Cu") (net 11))
 (segment (start 129.33 129.408) (end 129.33 128.545) (width 0.5) (layer "B.Cu") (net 11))
 (segment (start 131.5 127.475) (end 133 125.975) (width 0.5) (layer "B.Cu") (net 11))
 (segment (start 130.6 128.8) (end 131.185 128.215) (width 0.5) (layer "B.Cu") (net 10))
 (segment (start 134.05 126.45) (end 134.05 113.95) (width 0.5) (layer "B.Cu") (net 10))
 (segment (start 142.75 108.725) (end 147.6 103.875) (width 0.5) (layer "B.Cu") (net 10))
 (segment (start 134.05 113.95) (end 139.275 108.725) (width 0.5) (layer "B.Cu") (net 10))
 (segment (start 130.6 129.408) (end 130.6 128.8) (width 0.5) (layer "B.Cu") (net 10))
 (segment (start 147.6 103.875) (end 147.6 92.088) (width 0.5) (layer "B.Cu") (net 10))
 (segment (start 131.185 128.215) (end 132.285 128.215) (width 0.5) (layer "B.Cu") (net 10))
 (segment (start 147.6 92.088) (end 149.79 89.898) (width 0.5) (layer "B.Cu") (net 10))
 (segment (start 132.285 128.215) (end 134.05 126.45) (width 0.5) (layer "B.Cu") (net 10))
 (segment (start 139.275 108.725) (end 142.75 108.725) (width 0.5) (layer "B.Cu") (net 10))
 (segment (start 142.29 97.96) (end 142.29 89.898) (width 0.5) (layer "B.Cu") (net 13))
 (segment (start 124.1 116.15) (end 142.29 97.96) (width 0.5) (layer "B.Cu") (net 13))
 (segment (start 126.79 129.408) (end 126.79 129.14) (width 0.5) (layer "B.Cu") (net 13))
 (segment (start 126.79 129.14) (end 124.1 126.45) (width 0.5) (layer "B.Cu") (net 13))
 (segment (start 124.1 126.45) (end 124.1 116.15) (width 0.5) (layer "B.Cu") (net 13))
 (segment (start 127.925 124.45) (end 129.575 126.1) (width 0.5) (layer "F.Cu") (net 31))
 (segment (start 134.67 121.63) (end 135.705 121.63) (width 0.5) (layer "F.Cu") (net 31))
 (segment (start 131.525 126.1) (end 133.4 124.225) (width 0.5) (layer "F.Cu") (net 31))
 (segment (start 133.4 122.9) (end 134.67 121.63) (width 0.5) (layer "F.Cu") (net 31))
 (segment (start 133.4 124.225) (end 133.4 122.9) (width 0.5) (layer "F.Cu") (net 31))
 (segment (start 129.575 126.1) (end 131.525 126.1) (width 0.5) (layer "F.Cu") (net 31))
 (segment (start 134.34 123.585) (end 135.025 122.9) (width 0.5) (layer "F.Cu") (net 30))
 (segment (start 135.025 122.9) (end 135.705 122.9) (width 0.5) (layer "F.Cu") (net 30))
 (segment (start 134.34 124.685) (end 134.34 123.585) (width 0.5) (layer "F.Cu") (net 30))
 (segment (start 128 127.025) (end 132 127.025) (width 0.5) (layer "F.Cu") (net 30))
 (segment (start 132 127.025) (end 134.34 124.685) (width 0.5) (layer "F.Cu") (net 30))
 (segment (start 125.425 124.45) (end 128 127.025) (width 0.5) (layer "F.Cu") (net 30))
 (segment (start 124.85 94.94) (end 124.75 94.94) (width 0.5) (layer "F.Cu") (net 6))
 (segment (start 129.15 99.24) (end 124.85 94.94) (width 0.5) (layer "F.Cu") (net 6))
 (segment (start 120.223503 115.848) (end 129.15 106.921503) (width 0.5) (layer "B.Cu") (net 6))
 (segment (start 129.15 106.921503) (end 129.15 99.24) (width 0.5) (layer "B.Cu") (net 6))
 (segment (start 120.15 115.848) (end 120.223503 115.848) (width 0.5) (layer "B.Cu") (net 6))
 (segment (start 122.1 102.67) (end 124.75 100.02) (width 0.5) (layer "B.Cu") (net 8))
 (segment (start 120.15 109.498) (end 120.857106 109.498) (width 0.5) (layer "B.Cu") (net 8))
 (segment (start 122.1 108.255106) (end 122.1 102.67) (width 0.5) (layer "B.Cu") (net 8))
 (segment (start 120.857106 109.498) (end 122.1 108.255106) (width 0.5) (layer "B.Cu") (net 8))
 (segment (start 120.15 110.768) (end 120.857106 110.768) (width 0.5) (layer "B.Cu") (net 9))
 (segment (start 123.05 104.26) (end 124.75 102.56) (width 0.5) (layer "B.Cu") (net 9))
 (segment (start 120.857106 110.768) (end 123.05 108.575106) (width 0.5) (layer "B.Cu") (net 9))
 (segment (start 123.05 108.575106) (end 123.05 104.26) (width 0.5) (layer "B.Cu") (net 9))
 (segment (start 150.275 94.7075) (end 150.2675 94.7) (width 0.5) (layer "F.Cu") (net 14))
 (segment (start 150.275 97.65) (end 150.275 94.7075) (width 0.5) (layer "F.Cu") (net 14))
 (segment (start 140.79 116.3175) (end 140.79 113.6) (width 0.5) (layer "F.Cu") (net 18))
 (segment (start 140.7825 116.325) (end 140.79 116.3175) (width 0.25) (layer "F.Cu") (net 18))
 (segment (start 146.9825 102.725) (end 150.27 102.725) (width 0.5) (layer "F.Cu") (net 1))
 (segment (start 150.27 102.725) (end 150.275 102.73) (width 0.5) (layer "F.Cu") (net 1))
 (segment (start 129.15 96.7) (end 129.15 94.3925) (width 0.5) (layer "F.Cu") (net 19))
 (segment (start 129.15 94.3925) (end 129.1325 94.375) (width 0.5) (layer "F.Cu") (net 19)))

